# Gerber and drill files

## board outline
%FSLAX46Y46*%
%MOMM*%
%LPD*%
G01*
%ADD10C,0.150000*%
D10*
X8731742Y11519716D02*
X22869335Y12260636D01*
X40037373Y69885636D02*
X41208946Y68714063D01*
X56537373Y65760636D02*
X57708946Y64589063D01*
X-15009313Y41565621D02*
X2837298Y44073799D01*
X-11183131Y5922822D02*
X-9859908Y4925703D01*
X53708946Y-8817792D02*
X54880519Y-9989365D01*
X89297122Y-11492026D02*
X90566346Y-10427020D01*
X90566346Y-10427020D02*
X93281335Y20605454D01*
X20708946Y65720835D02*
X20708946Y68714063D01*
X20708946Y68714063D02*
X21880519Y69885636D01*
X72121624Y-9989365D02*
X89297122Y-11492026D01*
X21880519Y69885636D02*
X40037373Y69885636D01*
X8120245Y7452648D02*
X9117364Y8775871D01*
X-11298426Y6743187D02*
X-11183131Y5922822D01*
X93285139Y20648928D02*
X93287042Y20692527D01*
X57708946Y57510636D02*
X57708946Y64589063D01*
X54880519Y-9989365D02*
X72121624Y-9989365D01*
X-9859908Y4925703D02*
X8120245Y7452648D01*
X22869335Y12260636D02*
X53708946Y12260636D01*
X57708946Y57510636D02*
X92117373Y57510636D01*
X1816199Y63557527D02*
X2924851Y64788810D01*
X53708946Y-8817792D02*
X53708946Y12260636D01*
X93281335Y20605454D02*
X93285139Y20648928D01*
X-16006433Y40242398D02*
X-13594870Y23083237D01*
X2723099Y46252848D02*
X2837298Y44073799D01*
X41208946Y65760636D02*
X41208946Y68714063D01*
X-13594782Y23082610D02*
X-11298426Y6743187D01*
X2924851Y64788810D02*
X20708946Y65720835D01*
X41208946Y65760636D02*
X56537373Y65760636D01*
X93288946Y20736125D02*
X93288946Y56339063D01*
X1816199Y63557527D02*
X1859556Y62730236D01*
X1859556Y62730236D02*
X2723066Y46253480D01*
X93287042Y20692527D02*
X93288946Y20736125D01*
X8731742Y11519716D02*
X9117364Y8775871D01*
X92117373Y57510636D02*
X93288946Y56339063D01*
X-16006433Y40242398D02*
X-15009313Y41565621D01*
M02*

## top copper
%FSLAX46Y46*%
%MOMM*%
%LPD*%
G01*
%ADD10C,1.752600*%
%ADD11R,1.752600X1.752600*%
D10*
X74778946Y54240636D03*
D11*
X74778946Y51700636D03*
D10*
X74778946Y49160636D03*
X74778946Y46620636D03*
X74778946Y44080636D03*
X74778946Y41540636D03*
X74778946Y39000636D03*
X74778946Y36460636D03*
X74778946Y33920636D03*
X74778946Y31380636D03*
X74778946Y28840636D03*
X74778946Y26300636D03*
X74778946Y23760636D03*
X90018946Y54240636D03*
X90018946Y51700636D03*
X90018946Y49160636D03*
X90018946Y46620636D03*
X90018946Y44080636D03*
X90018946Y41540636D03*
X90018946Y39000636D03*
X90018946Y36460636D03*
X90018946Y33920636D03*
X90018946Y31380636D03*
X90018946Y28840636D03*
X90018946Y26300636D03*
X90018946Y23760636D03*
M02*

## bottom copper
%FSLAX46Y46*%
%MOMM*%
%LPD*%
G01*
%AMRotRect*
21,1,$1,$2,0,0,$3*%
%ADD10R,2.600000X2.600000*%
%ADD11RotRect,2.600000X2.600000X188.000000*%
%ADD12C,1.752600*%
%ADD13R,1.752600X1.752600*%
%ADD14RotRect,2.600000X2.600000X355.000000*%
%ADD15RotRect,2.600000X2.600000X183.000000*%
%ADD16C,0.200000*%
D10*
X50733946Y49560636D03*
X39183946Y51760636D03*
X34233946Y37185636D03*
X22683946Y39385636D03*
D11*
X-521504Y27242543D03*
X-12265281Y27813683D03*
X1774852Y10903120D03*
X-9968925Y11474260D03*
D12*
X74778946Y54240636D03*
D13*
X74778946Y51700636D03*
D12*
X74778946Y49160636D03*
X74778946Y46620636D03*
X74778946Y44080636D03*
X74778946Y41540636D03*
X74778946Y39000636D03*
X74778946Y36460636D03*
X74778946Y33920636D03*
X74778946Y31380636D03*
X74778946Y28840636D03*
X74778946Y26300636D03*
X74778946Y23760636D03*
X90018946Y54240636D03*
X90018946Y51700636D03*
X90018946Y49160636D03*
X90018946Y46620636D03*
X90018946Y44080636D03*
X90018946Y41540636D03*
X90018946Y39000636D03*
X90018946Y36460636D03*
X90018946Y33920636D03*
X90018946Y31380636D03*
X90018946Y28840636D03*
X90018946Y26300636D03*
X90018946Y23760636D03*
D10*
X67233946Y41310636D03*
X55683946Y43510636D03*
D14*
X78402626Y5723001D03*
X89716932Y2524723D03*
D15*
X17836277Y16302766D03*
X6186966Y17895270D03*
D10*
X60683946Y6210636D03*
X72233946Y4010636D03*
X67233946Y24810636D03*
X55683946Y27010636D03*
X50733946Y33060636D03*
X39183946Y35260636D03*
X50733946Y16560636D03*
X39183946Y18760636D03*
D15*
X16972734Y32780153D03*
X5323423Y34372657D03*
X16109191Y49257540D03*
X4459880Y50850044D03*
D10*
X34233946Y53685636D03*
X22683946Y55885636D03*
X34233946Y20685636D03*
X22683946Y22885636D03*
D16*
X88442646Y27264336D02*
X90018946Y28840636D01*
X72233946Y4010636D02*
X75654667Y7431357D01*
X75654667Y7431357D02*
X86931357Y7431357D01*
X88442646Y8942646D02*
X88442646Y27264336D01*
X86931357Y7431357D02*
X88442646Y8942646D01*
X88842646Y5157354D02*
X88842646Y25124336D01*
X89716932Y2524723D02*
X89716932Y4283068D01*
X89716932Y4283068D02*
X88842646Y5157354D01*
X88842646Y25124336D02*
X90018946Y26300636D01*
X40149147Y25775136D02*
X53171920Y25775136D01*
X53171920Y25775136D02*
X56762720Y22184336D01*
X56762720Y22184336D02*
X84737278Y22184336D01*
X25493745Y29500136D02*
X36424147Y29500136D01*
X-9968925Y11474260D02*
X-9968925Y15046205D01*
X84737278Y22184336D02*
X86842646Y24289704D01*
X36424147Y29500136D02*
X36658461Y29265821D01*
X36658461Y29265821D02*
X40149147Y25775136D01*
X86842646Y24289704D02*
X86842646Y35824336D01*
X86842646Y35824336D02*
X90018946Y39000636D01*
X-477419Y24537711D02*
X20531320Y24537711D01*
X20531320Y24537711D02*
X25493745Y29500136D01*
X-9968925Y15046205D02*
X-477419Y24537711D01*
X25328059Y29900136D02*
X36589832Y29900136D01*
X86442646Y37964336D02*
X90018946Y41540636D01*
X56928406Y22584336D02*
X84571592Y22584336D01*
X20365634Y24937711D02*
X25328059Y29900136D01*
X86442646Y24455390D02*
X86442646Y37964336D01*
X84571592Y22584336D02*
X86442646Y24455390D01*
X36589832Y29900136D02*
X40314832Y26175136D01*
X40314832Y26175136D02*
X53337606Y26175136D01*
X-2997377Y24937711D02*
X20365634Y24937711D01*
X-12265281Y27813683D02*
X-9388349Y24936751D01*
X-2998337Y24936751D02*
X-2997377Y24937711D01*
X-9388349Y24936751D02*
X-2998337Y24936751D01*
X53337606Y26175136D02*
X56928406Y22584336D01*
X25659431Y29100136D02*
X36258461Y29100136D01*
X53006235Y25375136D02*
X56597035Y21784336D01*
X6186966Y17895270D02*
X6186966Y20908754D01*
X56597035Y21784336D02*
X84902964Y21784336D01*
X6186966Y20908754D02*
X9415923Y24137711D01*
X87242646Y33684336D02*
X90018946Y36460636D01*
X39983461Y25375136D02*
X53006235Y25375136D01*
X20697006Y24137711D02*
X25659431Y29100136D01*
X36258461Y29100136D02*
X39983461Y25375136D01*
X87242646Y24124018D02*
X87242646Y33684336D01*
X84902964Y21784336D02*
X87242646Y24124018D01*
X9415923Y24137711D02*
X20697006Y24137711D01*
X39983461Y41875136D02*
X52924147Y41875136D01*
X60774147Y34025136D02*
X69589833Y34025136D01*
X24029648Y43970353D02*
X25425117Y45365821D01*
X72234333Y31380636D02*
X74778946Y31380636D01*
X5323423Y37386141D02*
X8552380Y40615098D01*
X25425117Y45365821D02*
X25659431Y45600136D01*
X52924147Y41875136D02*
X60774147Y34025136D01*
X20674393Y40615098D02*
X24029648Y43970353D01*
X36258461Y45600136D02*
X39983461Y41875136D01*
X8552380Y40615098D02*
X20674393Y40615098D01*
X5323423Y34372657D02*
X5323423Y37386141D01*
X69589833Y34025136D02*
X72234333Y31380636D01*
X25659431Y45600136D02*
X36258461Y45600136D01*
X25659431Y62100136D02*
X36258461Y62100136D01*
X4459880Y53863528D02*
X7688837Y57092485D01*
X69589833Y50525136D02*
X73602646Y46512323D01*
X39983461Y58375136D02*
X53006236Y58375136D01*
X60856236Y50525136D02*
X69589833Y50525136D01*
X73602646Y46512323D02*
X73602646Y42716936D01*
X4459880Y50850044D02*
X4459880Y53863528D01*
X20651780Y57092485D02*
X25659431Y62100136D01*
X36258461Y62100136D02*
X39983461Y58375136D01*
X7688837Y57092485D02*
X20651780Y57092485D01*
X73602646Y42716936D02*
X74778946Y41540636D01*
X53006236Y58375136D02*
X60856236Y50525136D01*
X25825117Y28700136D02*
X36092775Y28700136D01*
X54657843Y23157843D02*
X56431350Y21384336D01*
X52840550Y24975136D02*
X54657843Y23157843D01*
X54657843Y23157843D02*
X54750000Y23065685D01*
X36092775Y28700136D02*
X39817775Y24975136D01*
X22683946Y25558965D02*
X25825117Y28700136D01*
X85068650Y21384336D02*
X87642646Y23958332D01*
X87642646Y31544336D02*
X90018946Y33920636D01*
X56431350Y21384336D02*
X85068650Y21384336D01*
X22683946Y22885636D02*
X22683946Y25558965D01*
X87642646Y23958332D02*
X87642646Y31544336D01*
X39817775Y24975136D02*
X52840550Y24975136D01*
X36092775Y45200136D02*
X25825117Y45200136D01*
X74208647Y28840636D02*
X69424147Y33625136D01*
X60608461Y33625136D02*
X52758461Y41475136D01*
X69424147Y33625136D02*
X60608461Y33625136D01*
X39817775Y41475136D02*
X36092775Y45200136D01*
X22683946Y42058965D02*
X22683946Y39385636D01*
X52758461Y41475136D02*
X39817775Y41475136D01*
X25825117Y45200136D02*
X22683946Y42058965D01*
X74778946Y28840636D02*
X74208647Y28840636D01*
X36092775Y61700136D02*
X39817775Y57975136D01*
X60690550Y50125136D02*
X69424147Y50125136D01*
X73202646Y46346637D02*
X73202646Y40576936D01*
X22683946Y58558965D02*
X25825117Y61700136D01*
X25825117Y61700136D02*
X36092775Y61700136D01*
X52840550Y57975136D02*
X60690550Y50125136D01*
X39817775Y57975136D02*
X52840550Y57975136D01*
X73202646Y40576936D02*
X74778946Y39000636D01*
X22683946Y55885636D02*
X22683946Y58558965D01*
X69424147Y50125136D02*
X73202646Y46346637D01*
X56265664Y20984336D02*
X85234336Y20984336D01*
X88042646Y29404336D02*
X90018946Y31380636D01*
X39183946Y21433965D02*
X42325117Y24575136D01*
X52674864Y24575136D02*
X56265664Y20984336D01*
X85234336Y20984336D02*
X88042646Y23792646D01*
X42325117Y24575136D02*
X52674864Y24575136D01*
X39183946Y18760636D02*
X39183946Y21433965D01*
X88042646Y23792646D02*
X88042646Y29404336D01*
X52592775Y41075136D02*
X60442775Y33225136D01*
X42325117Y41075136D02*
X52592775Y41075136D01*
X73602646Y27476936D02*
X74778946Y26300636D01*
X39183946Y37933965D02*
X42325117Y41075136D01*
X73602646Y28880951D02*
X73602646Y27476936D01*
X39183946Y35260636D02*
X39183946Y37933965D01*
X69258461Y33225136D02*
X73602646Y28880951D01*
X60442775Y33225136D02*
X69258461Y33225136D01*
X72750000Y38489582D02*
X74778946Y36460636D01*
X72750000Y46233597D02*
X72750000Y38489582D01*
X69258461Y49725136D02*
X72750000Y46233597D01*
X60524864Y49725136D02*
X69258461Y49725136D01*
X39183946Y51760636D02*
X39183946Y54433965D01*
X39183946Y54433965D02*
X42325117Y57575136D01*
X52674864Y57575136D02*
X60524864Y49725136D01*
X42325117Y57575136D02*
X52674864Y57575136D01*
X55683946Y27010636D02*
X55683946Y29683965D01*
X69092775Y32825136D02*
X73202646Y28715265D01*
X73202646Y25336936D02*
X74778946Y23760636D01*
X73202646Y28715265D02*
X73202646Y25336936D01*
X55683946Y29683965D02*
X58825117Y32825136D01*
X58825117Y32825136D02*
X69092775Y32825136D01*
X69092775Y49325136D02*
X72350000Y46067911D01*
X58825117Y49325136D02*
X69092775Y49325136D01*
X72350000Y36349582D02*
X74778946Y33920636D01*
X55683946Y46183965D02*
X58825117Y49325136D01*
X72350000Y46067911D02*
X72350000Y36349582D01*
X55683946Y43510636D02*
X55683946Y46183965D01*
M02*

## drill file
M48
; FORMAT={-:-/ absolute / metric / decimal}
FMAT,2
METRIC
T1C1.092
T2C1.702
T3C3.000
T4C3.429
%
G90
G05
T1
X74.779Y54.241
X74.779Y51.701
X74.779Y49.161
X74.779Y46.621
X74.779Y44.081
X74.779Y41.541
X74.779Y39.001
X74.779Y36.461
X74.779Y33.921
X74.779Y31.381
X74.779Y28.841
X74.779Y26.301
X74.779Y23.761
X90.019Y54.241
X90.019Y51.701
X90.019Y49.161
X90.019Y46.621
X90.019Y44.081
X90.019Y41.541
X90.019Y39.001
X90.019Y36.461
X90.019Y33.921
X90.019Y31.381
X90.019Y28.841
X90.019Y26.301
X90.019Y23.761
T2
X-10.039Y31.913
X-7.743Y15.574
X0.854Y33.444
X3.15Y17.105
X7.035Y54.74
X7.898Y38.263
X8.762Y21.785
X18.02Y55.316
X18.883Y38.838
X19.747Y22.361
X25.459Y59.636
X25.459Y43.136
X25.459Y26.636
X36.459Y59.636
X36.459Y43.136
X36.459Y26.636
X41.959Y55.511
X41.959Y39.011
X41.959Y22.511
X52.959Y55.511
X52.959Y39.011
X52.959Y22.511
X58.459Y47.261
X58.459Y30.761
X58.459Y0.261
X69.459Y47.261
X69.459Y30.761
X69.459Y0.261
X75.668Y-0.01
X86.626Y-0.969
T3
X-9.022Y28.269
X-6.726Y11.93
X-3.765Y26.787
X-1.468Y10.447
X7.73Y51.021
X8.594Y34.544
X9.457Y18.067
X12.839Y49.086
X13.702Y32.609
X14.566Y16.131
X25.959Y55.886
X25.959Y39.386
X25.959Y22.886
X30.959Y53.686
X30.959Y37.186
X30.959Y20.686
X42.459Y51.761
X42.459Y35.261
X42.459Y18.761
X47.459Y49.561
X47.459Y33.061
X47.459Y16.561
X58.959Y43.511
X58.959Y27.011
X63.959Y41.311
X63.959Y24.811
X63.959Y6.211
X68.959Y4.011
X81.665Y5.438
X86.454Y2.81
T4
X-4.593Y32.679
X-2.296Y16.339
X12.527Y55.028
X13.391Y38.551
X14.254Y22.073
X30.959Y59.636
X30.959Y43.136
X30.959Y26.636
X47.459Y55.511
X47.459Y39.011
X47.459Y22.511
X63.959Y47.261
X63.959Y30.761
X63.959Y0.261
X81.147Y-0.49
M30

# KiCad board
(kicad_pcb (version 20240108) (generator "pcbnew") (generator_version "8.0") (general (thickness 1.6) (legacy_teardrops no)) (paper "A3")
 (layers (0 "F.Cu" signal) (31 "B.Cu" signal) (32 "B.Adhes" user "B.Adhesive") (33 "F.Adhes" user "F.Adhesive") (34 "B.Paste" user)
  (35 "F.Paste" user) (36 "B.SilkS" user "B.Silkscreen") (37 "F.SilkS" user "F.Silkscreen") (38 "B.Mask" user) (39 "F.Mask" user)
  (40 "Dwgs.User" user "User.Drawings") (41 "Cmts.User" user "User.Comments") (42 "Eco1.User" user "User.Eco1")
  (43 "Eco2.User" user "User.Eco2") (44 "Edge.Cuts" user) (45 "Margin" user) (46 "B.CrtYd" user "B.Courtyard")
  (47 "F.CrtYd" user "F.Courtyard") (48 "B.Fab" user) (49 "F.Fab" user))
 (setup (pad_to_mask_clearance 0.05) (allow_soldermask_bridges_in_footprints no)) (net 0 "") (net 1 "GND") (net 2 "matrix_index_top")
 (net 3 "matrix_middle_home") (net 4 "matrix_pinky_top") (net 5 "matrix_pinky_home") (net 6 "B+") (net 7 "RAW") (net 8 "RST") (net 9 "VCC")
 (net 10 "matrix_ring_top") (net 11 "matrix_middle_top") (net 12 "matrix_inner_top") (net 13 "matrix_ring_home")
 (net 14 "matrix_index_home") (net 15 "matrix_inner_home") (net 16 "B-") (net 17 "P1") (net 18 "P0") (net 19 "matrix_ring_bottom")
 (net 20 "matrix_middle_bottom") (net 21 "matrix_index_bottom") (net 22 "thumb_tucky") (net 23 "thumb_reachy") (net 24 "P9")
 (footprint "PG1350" (layer "F.Cu") (at 47.458946 -55.510636 180)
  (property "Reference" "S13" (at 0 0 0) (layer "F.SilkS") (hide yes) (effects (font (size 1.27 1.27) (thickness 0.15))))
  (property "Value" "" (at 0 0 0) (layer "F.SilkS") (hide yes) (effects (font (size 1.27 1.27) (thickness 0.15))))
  (pad "" np_thru_hole circle (at -5.5 0) (size 1.7018 1.7018) (drill 1.7018) (layers "*.Cu" "*.Mask"))
  (pad "" np_thru_hole circle (at 0 -5.95) (size 3 3) (drill 3) (layers "*.Cu" "*.Mask"))
  (pad "" np_thru_hole circle (at 0 0) (size 3.429 3.429) (drill 3.429) (layers "*.Cu" "*.Mask"))
  (pad "" np_thru_hole circle (at 5 -3.75) (size 3 3) (drill 3) (layers "*.Cu" "*.Mask"))
  (pad "" np_thru_hole circle (at 5.5 0) (size 1.7018 1.7018) (drill 1.7018) (layers "*.Cu" "*.Mask"))
  (pad "1" smd rect (at -3.275 -5.95 180) (size 2.6 2.6) (layers "B.Cu" "B.Paste" "B.Mask") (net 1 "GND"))
  (pad "2" smd rect (at 8.275 -3.75 180) (size 2.6 2.6) (layers "B.Cu" "B.Paste" "B.Mask") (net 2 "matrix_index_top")))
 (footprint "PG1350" (layer "F.Cu") (at 30.958946 -43.135636 180)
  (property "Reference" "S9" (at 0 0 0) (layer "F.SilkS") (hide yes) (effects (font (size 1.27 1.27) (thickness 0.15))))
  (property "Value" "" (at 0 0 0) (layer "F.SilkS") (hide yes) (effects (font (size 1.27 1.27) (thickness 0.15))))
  (pad "" np_thru_hole circle (at -5.5 0) (size 1.7018 1.7018) (drill 1.7018) (layers "*.Cu" "*.Mask"))
  (pad "" np_thru_hole circle (at 0 -5.95) (size 3 3) (drill 3) (layers "*.Cu" "*.Mask"))
  (pad "" np_thru_hole circle (at 0 0) (size 3.429 3.429) (drill 3.429) (layers "*.Cu" "*.Mask"))
  (pad "" np_thru_hole circle (at 5 -3.75) (size 3 3) (drill 3) (layers "*.Cu" "*.Mask"))
  (pad "" np_thru_hole circle (at 5.5 0) (size 1.7018 1.7018) (drill 1.7018) (layers "*.Cu" "*.Mask"))
  (pad "1" smd rect (at -3.275 -5.95 180) (size 2.6 2.6) (layers "B.Cu" "B.Paste" "B.Mask") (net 1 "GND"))
  (pad "2" smd rect (at 8.275 -3.75 180) (size 2.6 2.6) (layers "B.Cu" "B.Paste" "B.Mask") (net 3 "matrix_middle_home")))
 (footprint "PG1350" (layer "F.Cu") (at -4.592712 -32.678846 -172)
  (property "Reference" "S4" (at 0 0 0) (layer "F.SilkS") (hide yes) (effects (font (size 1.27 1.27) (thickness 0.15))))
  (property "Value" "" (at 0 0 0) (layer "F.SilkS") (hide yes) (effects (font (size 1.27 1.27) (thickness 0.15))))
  (pad "" np_thru_hole circle (at -5.5 0) (size 1.7018 1.7018) (drill 1.7018) (layers "*.Cu" "*.Mask"))
  (pad "" np_thru_hole circle (at 0 -5.95) (size 3 3) (drill 3) (layers "*.Cu" "*.Mask"))
  (pad "" np_thru_hole circle (at 0 0) (size 3.429 3.429) (drill 3.429) (layers "*.Cu" "*.Mask"))
  (pad "" np_thru_hole circle (at 5 -3.75) (size 3 3) (drill 3) (layers "*.Cu" "*.Mask"))
  (pad "" np_thru_hole circle (at 5.5 0) (size 1.7018 1.7018) (drill 1.7018) (layers "*.Cu" "*.Mask"))
  (pad "1" smd rect (at -3.275 -5.95 188) (size 2.6 2.6) (layers "B.Cu" "B.Paste" "B.Mask") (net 1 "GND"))
  (pad "2" smd rect (at 8.275 -3.75 188) (size 2.6 2.6) (layers "B.Cu" "B.Paste" "B.Mask") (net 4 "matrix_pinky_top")))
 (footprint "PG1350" (layer "F.Cu") (at -2.296356 -16.339423 -172)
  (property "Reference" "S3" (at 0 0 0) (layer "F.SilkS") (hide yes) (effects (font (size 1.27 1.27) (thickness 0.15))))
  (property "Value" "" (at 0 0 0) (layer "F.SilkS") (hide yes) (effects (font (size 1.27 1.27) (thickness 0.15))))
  (pad "" np_thru_hole circle (at -5.5 0) (size 1.7018 1.7018) (drill 1.7018) (layers "*.Cu" "*.Mask"))
  (pad "" np_thru_hole circle (at 0 -5.95) (size 3 3) (drill 3) (layers "*.Cu" "*.Mask"))
  (pad "" np_thru_hole circle (at 0 0) (size 3.429 3.429) (drill 3.429) (layers "*.Cu" "*.Mask"))
  (pad "" np_thru_hole circle (at 5 -3.75) (size 3 3) (drill 3) (layers "*.Cu" "*.Mask"))
  (pad "" np_thru_hole circle (at 5.5 0) (size 1.7018 1.7018) (drill 1.7018) (layers "*.Cu" "*.Mask"))
  (pad "1" smd rect (at -3.275 -5.95 188) (size 2.6 2.6) (layers "B.Cu" "B.Paste" "B.Mask") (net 1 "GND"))
  (pad "2" smd rect (at 8.275 -3.75 188) (size 2.6 2.6) (layers "B.Cu" "B.Paste" "B.Mask") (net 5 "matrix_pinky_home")))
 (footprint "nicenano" (layer "F.Cu") (at 82.398946 -39.000636 -90)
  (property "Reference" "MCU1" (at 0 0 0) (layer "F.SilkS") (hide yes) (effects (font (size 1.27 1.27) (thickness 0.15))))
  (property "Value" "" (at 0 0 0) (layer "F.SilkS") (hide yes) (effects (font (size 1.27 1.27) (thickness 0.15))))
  (pad "1" thru_hole circle (at -15.24 7.62) (size 1.7526 1.7526) (drill 1.0922) (layers "*.Cu" "*.SilkS" "*.Mask")
   (remove_unused_layers no) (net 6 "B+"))
  (pad "2" thru_hole rect (at -12.7 7.62 270) (size 1.7526 1.7526) (drill 1.0922) (layers "*.Cu" "*.SilkS" "*.Mask")
   (remove_unused_layers no) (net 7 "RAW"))
  (pad "3" thru_hole circle (at -10.16 7.62) (size 1.7526 1.7526) (drill 1.0922) (layers "*.Cu" "*.SilkS" "*.Mask")
   (remove_unused_layers no) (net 1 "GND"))
  (pad "4" thru_hole circle (at -7.62 7.62) (size 1.7526 1.7526) (drill 1.0922) (layers "*.Cu" "*.SilkS" "*.Mask") (remove_unused_layers no)
   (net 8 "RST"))
  (pad "5" thru_hole circle (at -5.08 7.62) (size 1.7526 1.7526) (drill 1.0922) (layers "*.Cu" "*.SilkS" "*.Mask") (remove_unused_layers no)
   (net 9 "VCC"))
  (pad "6" thru_hole circle (at -2.54 7.62) (size 1.7526 1.7526) (drill 1.0922) (layers "*.Cu" "*.SilkS" "*.Mask") (remove_unused_layers no)
   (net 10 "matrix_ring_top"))
  (pad "7" thru_hole circle (at 0 7.62) (size 1.7526 1.7526) (drill 1.0922) (layers "*.Cu" "*.SilkS" "*.Mask") (remove_unused_layers no)
   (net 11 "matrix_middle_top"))
  (pad "8" thru_hole circle (at 2.54 7.62) (size 1.7526 1.7526) (drill 1.0922) (layers "*.Cu" "*.SilkS" "*.Mask") (remove_unused_layers no)
   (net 2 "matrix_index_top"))
  (pad "9" thru_hole circle (at 5.08 7.62) (size 1.7526 1.7526) (drill 1.0922) (layers "*.Cu" "*.SilkS" "*.Mask") (remove_unused_layers no)
   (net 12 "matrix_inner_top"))
  (pad "10" thru_hole circle (at 7.62 7.62) (size 1.7526 1.7526) (drill 1.0922) (layers "*.Cu" "*.SilkS" "*.Mask") (remove_unused_layers no)
   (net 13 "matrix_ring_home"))
  (pad "11" thru_hole circle (at 10.16 7.62) (size 1.7526 1.7526) (drill 1.0922) (layers "*.Cu" "*.SilkS" "*.Mask")
   (remove_unused_layers no) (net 3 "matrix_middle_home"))
  (pad "12" thru_hole circle (at 12.7 7.62) (size 1.7526 1.7526) (drill 1.0922) (layers "*.Cu" "*.SilkS" "*.Mask") (remove_unused_layers no)
   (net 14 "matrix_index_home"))
  (pad "13" thru_hole circle (at 15.24 7.62) (size 1.7526 1.7526) (drill 1.0922) (layers "*.Cu" "*.SilkS" "*.Mask")
   (remove_unused_layers no) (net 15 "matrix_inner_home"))
  (pad "14" thru_hole circle (at -15.24 -7.62) (size 1.7526 1.7526) (drill 1.0922) (layers "*.Cu" "*.SilkS" "*.Mask")
   (remove_unused_layers no) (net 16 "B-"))
  (pad "15" thru_hole circle (at -12.7 -7.62) (size 1.7526 1.7526) (drill 1.0922) (layers "*.Cu" "*.SilkS" "*.Mask")
   (remove_unused_layers no) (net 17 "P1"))
  (pad "16" thru_hole circle (at -10.16 -7.62) (size 1.7526 1.7526) (drill 1.0922) (layers "*.Cu" "*.SilkS" "*.Mask")
   (remove_unused_layers no) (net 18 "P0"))
  (pad "17" thru_hole circle (at -7.62 -7.62) (size 1.7526 1.7526) (drill 1.0922) (layers "*.Cu" "*.SilkS" "*.Mask")
   (remove_unused_layers no) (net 1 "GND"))
  (pad "18" thru_hole circle (at -5.08 -7.62) (size 1.7526 1.7526) (drill 1.0922) (layers "*.Cu" "*.SilkS" "*.Mask")
   (remove_unused_layers no) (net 1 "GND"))
  (pad "19" thru_hole circle (at -2.54 -7.62) (size 1.7526 1.7526) (drill 1.0922) (layers "*.Cu" "*.SilkS" "*.Mask")
   (remove_unused_layers no) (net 4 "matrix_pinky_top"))
  (pad "20" thru_hole circle (at 0 -7.62) (size 1.7526 1.7526) (drill 1.0922) (layers "*.Cu" "*.SilkS" "*.Mask") (remove_unused_layers no)
   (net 5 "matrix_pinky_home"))
  (pad "21" thru_hole circle (at 2.54 -7.62) (size 1.7526 1.7526) (drill 1.0922) (layers "*.Cu" "*.SilkS" "*.Mask")
   (remove_unused_layers no) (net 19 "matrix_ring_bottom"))
  (pad "22" thru_hole circle (at 5.08 -7.62) (size 1.7526 1.7526) (drill 1.0922) (layers "*.Cu" "*.SilkS" "*.Mask")
   (remove_unused_layers no) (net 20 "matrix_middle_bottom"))
  (pad "23" thru_hole circle (at 7.62 -7.62) (size 1.7526 1.7526) (drill 1.0922) (layers "*.Cu" "*.SilkS" "*.Mask")
   (remove_unused_layers no) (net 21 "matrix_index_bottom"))
  (pad "24" thru_hole circle (at 10.16 -7.62) (size 1.7526 1.7526) (drill 1.0922) (layers "*.Cu" "*.SilkS" "*.Mask")
   (remove_unused_layers no) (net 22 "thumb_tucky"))
  (pad "25" thru_hole circle (at 12.7 -7.62) (size 1.7526 1.7526) (drill 1.0922) (layers "*.Cu" "*.SilkS" "*.Mask")
   (remove_unused_layers no) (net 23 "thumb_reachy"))
  (pad "26" thru_hole circle (at 15.24 -7.62) (size 1.7526 1.7526) (drill 1.0922) (layers "*.Cu" "*.SilkS" "*.Mask")
   (remove_unused_layers no) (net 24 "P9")))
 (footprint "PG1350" (layer "F.Cu") (at 63.958946 -47.260636 180)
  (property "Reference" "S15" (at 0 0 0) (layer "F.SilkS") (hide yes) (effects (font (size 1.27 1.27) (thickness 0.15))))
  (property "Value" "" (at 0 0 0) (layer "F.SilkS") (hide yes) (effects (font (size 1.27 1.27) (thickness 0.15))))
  (pad "" np_thru_hole circle (at -5.5 0) (size 1.7018 1.7018) (drill 1.7018) (layers "*.Cu" "*.Mask"))
  (pad "" np_thru_hole circle (at 0 -5.95) (size 3 3) (drill 3) (layers "*.Cu" "*.Mask"))
  (pad "" np_thru_hole circle (at 0 0) (size 3.429 3.429) (drill 3.429) (layers "*.Cu" "*.Mask"))
  (pad "" np_thru_hole circle (at 5 -3.75) (size 3 3) (drill 3) (layers "*.Cu" "*.Mask"))
  (pad "" np_thru_hole circle (at 5.5 0) (size 1.7018 1.7018) (drill 1.7018) (layers "*.Cu" "*.Mask"))
  (pad "1" smd rect (at -3.275 -5.95 180) (size 2.6 2.6) (layers "B.Cu" "B.Paste" "B.Mask") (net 1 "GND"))
  (pad "2" smd rect (at 8.275 -3.75 180) (size 2.6 2.6) (layers "B.Cu" "B.Paste" "B.Mask") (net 12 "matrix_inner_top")))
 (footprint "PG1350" (layer "F.Cu") (at 81.146587 0.489793 -5)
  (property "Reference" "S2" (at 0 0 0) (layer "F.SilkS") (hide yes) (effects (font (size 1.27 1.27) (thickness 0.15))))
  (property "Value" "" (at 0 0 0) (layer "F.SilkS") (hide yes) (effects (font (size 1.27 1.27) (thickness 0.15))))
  (pad "" np_thru_hole circle (at -5.5 0) (size 1.7018 1.7018) (drill 1.7018) (layers "*.Cu" "*.Mask"))
  (pad "" np_thru_hole circle (at 0 -5.95) (size 3 3) (drill 3) (layers "*.Cu" "*.Mask"))
  (pad "" np_thru_hole circle (at 0 0) (size 3.429 3.429) (drill 3.429) (layers "*.Cu" "*.Mask"))
  (pad "" np_thru_hole circle (at 5.000001 -3.75) (size 3 3) (drill 3) (layers "*.Cu" "*.Mask"))
  (pad "" np_thru_hole circle (at 5.5 0) (size 1.7018 1.7018) (drill 1.7018) (layers "*.Cu" "*.Mask"))
  (pad "1" smd rect (at -3.275 -5.95 355) (size 2.6 2.6) (layers "B.Cu" "B.Paste" "B.Mask") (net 1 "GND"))
  (pad "2" smd rect (at 8.275 -3.75 355) (size 2.6 2.6) (layers "B.Cu" "B.Paste" "B.Mask") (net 23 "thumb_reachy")))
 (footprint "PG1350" (layer "F.Cu") (at 14.254366 -22.073211 -177)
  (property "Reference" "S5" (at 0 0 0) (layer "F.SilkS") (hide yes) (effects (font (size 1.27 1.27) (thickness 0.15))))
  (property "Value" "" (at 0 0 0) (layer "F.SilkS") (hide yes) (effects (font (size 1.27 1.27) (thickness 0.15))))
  (pad "" np_thru_hole circle (at -5.5 0) (size 1.7018 1.7018) (drill 1.7018) (layers "*.Cu" "*.Mask"))
  (pad "" np_thru_hole circle (at 0 -5.95) (size 3 3) (drill 3) (layers "*.Cu" "*.Mask"))
  (pad "" np_thru_hole circle (at 0 0) (size 3.429 3.429) (drill 3.429) (layers "*.Cu" "*.Mask"))
  (pad "" np_thru_hole circle (at 5 -3.75) (size 3 3) (drill 3) (layers "*.Cu" "*.Mask"))
  (pad "" np_thru_hole circle (at 5.5 0) (size 1.7018 1.7018) (drill 1.7018) (layers "*.Cu" "*.Mask"))
  (pad "1" smd rect (at -3.275 -5.95 183) (size 2.6 2.6) (layers "B.Cu" "B.Paste" "B.Mask") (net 1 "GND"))
  (pad "2" smd rect (at 8.275 -3.75 183) (size 2.6 2.6) (layers "B.Cu" "B.Paste" "B.Mask") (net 19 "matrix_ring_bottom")))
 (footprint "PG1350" (layer "F.Cu") (at 63.958946 -0.260636)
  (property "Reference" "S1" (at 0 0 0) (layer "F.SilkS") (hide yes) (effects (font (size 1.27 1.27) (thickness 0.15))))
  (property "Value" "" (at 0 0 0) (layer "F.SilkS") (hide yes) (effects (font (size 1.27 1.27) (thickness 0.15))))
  (pad "" np_thru_hole circle (at -5.5 0) (size 1.7018 1.7018) (drill 1.7018) (layers "*.Cu" "*.Mask"))
  (pad "" np_thru_hole circle (at 0 -5.95) (size 3 3) (drill 3) (layers "*.Cu" "*.Mask"))
  (pad "" np_thru_hole circle (at 0 0) (size 3.429 3.429) (drill 3.429) (layers "*.Cu" "*.Mask"))
  (pad "" np_thru_hole circle (at 5 -3.75) (size 3 3) (drill 3) (layers "*.Cu" "*.Mask"))
  (pad "" np_thru_hole circle (at 5.5 0) (size 1.7018 1.7018) (drill 1.7018) (layers "*.Cu" "*.Mask"))
  (pad "1" smd rect (at -3.275 -5.95) (size 2.6 2.6) (layers "B.Cu" "B.Paste" "B.Mask") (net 1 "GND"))
  (pad "2" smd rect (at 8.275 -3.75) (size 2.6 2.6) (layers "B.Cu" "B.Paste" "B.Mask") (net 22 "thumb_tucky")))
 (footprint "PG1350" (layer "F.Cu") (at 63.958946 -30.760636 180)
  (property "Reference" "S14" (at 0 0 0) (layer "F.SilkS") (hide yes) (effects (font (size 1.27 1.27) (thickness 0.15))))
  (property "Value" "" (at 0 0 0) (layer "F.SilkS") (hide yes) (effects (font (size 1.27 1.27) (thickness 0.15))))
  (pad "" np_thru_hole circle (at -5.5 0) (size 1.7018 1.7018) (drill 1.7018) (layers "*.Cu" "*.Mask"))
  (pad "" np_thru_hole circle (at 0 -5.95) (size 3 3) (drill 3) (layers "*.Cu" "*.Mask"))
  (pad "" np_thru_hole circle (at 0 0) (size 3.429 3.429) (drill 3.429) (layers "*.Cu" "*.Mask"))
  (pad "" np_thru_hole circle (at 5 -3.75) (size 3 3) (drill 3) (layers "*.Cu" "*.Mask"))
  (pad "" np_thru_hole circle (at 5.5 0) (size 1.7018 1.7018) (drill 1.7018) (layers "*.Cu" "*.Mask"))
  (pad "1" smd rect (at -3.275 -5.95 180) (size 2.6 2.6) (layers "B.Cu" "B.Paste" "B.Mask") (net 1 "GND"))
  (pad "2" smd rect (at 8.275 -3.75 180) (size 2.6 2.6) (layers "B.Cu" "B.Paste" "B.Mask") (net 15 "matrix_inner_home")))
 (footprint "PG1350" (layer "F.Cu") (at 47.458946 -39.010636 180)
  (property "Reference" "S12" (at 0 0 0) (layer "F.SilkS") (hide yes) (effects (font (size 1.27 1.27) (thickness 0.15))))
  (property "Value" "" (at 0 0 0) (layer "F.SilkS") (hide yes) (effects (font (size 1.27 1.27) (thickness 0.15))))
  (pad "" np_thru_hole circle (at -5.5 0) (size 1.7018 1.7018) (drill 1.7018) (layers "*.Cu" "*.Mask"))
  (pad "" np_thru_hole circle (at 0 -5.95) (size 3 3) (drill 3) (layers "*.Cu" "*.Mask"))
  (pad "" np_thru_hole circle (at 0 0) (size 3.429 3.429) (drill 3.429) (layers "*.Cu" "*.Mask"))
  (pad "" np_thru_hole circle (at 5 -3.75) (size 3 3) (drill 3) (layers "*.Cu" "*.Mask"))
  (pad "" np_thru_hole circle (at 5.5 0) (size 1.7018 1.7018) (drill 1.7018) (layers "*.Cu" "*.Mask"))
  (pad "1" smd rect (at -3.275 -5.95 180) (size 2.6 2.6) (layers "B.Cu" "B.Paste" "B.Mask") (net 1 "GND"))
  (pad "2" smd rect (at 8.275 -3.75 180) (size 2.6 2.6) (layers "B.Cu" "B.Paste" "B.Mask") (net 14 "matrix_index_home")))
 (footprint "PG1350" (layer "F.Cu") (at 47.458946 -22.510636 180)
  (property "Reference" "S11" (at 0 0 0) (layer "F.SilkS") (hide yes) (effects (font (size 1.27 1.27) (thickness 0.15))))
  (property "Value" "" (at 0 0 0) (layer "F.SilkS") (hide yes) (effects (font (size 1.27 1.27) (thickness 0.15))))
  (pad "" np_thru_hole circle (at -5.5 0) (size 1.7018 1.7018) (drill 1.7018) (layers "*.Cu" "*.Mask"))
  (pad "" np_thru_hole circle (at 0 -5.95) (size 3 3) (drill 3) (layers "*.Cu" "*.Mask"))
  (pad "" np_thru_hole circle (at 0 0) (size 3.429 3.429) (drill 3.429) (layers "*.Cu" "*.Mask"))
  (pad "" np_thru_hole circle (at 5 -3.75) (size 3 3) (drill 3) (layers "*.Cu" "*.Mask"))
  (pad "" np_thru_hole circle (at 5.5 0) (size 1.7018 1.7018) (drill 1.7018) (layers "*.Cu" "*.Mask"))
  (pad "1" smd rect (at -3.275 -5.95 180) (size 2.6 2.6) (layers "B.Cu" "B.Paste" "B.Mask") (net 1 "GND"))
  (pad "2" smd rect (at 8.275 -3.75 180) (size 2.6 2.6) (layers "B.Cu" "B.Paste" "B.Mask") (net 21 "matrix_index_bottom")))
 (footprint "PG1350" (layer "F.Cu") (at 13.390823 -38.550598 -177)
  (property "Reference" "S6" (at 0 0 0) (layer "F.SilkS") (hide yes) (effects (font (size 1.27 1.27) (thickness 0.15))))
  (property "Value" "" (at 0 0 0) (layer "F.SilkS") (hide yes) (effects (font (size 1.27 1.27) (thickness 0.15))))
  (pad "" np_thru_hole circle (at -5.5 0) (size 1.7018 1.7018) (drill 1.7018) (layers "*.Cu" "*.Mask"))
  (pad "" np_thru_hole circle (at 0 -5.95) (size 3 3) (drill 3) (layers "*.Cu" "*.Mask"))
  (pad "" np_thru_hole circle (at 0 0) (size 3.429 3.429) (drill 3.429) (layers "*.Cu" "*.Mask"))
  (pad "" np_thru_hole circle (at 5 -3.75) (size 3 3) (drill 3) (layers "*.Cu" "*.Mask"))
  (pad "" np_thru_hole circle (at 5.5 0) (size 1.7018 1.7018) (drill 1.7018) (layers "*.Cu" "*.Mask"))
  (pad "1" smd rect (at -3.275 -5.95 183) (size 2.6 2.6) (layers "B.Cu" "B.Paste" "B.Mask") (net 1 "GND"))
  (pad "2" smd rect (at 8.275 -3.75 183) (size 2.6 2.6) (layers "B.Cu" "B.Paste" "B.Mask") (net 13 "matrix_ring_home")))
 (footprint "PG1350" (layer "F.Cu") (at 12.52728 -55.027985 -177)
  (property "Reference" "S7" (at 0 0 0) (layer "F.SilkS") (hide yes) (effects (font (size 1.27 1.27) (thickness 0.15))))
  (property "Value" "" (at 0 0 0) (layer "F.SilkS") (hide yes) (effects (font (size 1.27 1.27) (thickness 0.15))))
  (pad "" np_thru_hole circle (at -5.5 0) (size 1.7018 1.7018) (drill 1.7018) (layers "*.Cu" "*.Mask"))
  (pad "" np_thru_hole circle (at 0 -5.95) (size 3 3) (drill 3) (layers "*.Cu" "*.Mask"))
  (pad "" np_thru_hole circle (at 0 0) (size 3.429 3.429) (drill 3.429) (layers "*.Cu" "*.Mask"))
  (pad "" np_thru_hole circle (at 5 -3.75) (size 3 3) (drill 3) (layers "*.Cu" "*.Mask"))
  (pad "" np_thru_hole circle (at 5.5 0) (size 1.7018 1.7018) (drill 1.7018) (layers "*.Cu" "*.Mask"))
  (pad "1" smd rect (at -3.275 -5.95 183) (size 2.6 2.6) (layers "B.Cu" "B.Paste" "B.Mask") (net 1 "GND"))
  (pad "2" smd rect (at 8.275 -3.75 183) (size 2.6 2.6) (layers "B.Cu" "B.Paste" "B.Mask") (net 10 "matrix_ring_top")))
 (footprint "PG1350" (layer "F.Cu") (at 30.958946 -59.635636 180)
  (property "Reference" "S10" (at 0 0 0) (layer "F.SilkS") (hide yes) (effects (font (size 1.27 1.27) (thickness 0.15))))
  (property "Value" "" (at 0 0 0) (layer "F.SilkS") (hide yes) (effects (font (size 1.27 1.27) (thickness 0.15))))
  (pad "" np_thru_hole circle (at -5.5 0) (size 1.7018 1.7018) (drill 1.7018) (layers "*.Cu" "*.Mask"))
  (pad "" np_thru_hole circle (at 0 -5.95) (size 3 3) (drill 3) (layers "*.Cu" "*.Mask"))
  (pad "" np_thru_hole circle (at 0 0) (size 3.429 3.429) (drill 3.429) (layers "*.Cu" "*.Mask"))
  (pad "" np_thru_hole circle (at 5 -3.75) (size 3 3) (drill 3) (layers "*.Cu" "*.Mask"))
  (pad "" np_thru_hole circle (at 5.5 0) (size 1.7018 1.7018) (drill 1.7018) (layers "*.Cu" "*.Mask"))
  (pad "1" smd rect (at -3.275 -5.95 180) (size 2.6 2.6) (layers "B.Cu" "B.Paste" "B.Mask") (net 1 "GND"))
  (pad "2" smd rect (at 8.275 -3.75 180) (size 2.6 2.6) (layers "B.Cu" "B.Paste" "B.Mask") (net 11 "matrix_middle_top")))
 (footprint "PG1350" (layer "F.Cu") (at 30.958946 -26.635636 180)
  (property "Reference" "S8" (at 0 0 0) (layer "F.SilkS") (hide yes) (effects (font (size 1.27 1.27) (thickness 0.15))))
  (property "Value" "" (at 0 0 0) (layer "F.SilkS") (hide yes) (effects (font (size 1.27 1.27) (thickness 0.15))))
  (pad "" np_thru_hole circle (at -5.5 0) (size 1.7018 1.7018) (drill 1.7018) (layers "*.Cu" "*.Mask"))
  (pad "" np_thru_hole circle (at 0 -5.95) (size 3 3) (drill 3) (layers "*.Cu" "*.Mask"))
  (pad "" np_thru_hole circle (at 0 0) (size 3.429 3.429) (drill 3.429) (layers "*.Cu" "*.Mask"))
  (pad "" np_thru_hole circle (at 5 -3.75) (size 3 3) (drill 3) (layers "*.Cu" "*.Mask"))
  (pad "" np_thru_hole circle (at 5.5 0) (size 1.7018 1.7018) (drill 1.7018) (layers "*.Cu" "*.Mask"))
  (pad "1" smd rect (at -3.275 -5.95 180) (size 2.6 2.6) (layers "B.Cu" "B.Paste" "B.Mask") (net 1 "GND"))
  (pad "2" smd rect (at 8.275 -3.75 180) (size 2.6 2.6) (layers "B.Cu" "B.Paste" "B.Mask") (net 20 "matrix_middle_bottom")))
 (gr_line (start 8.731742 -11.519716) (end 22.869335 -12.260636) (stroke (width 0.15) (type default)) (layer "Edge.Cuts"))
 (gr_line (start 40.037373 -69.885636) (end 41.208946 -68.714063) (stroke (width 0.15) (type default)) (layer "Edge.Cuts"))
 (gr_line (start 56.537373 -65.760636) (end 57.708946 -64.589063) (stroke (width 0.15) (type default)) (layer "Edge.Cuts"))
 (gr_line (start -15.009313 -41.565621) (end 2.837298 -44.073799) (stroke (width 0.15) (type default)) (layer "Edge.Cuts"))
 (gr_line (start -11.183131 -5.922822) (end -9.859908 -4.925703) (stroke (width 0.15) (type default)) (layer "Edge.Cuts"))
 (gr_line (start 53.708946 8.817792) (end 54.880519 9.989365) (stroke (width 0.15) (type default)) (layer "Edge.Cuts"))
 (gr_line (start 89.297122 11.492026) (end 90.566346 10.42702) (stroke (width 0.15) (type default)) (layer "Edge.Cuts"))
 (gr_line (start 90.566346 10.42702) (end 93.281335 -20.605454) (stroke (width 0.15) (type default)) (layer "Edge.Cuts"))
 (gr_line (start 20.708946 -65.720835) (end 20.708946 -68.714063) (stroke (width 0.15) (type default)) (layer "Edge.Cuts"))
 (gr_line (start 20.708946 -68.714063) (end 21.880519 -69.885636) (stroke (width 0.15) (type default)) (layer "Edge.Cuts"))
 (gr_line (start 72.121624 9.989365) (end 89.297122 11.492026) (stroke (width 0.15) (type default)) (layer "Edge.Cuts"))
 (gr_line (start 21.880519 -69.885636) (end 40.037373 -69.885636) (stroke (width 0.15) (type default)) (layer "Edge.Cuts"))
 (gr_line (start 8.120245 -7.452648) (end 9.117364 -8.775871) (stroke (width 0.15) (type default)) (layer "Edge.Cuts"))
 (gr_line (start -11.298426 -6.743187) (end -11.183131 -5.922822) (stroke (width 0.15) (type default)) (layer "Edge.Cuts"))
 (gr_line (start 93.285139 -20.648928) (end 93.287042 -20.692527) (stroke (width 0.15) (type default)) (layer "Edge.Cuts"))
 (gr_line (start 57.708946 -57.510636) (end 57.708946 -64.589063) (stroke (width 0.15) (type default)) (layer "Edge.Cuts"))
 (gr_line (start 54.880519 9.989365) (end 72.121624 9.989365) (stroke (width 0.15) (type default)) (layer "Edge.Cuts"))
 (gr_line (start -9.859908 -4.925703) (end 8.120245 -7.452648) (stroke (width 0.15) (type default)) (layer "Edge.Cuts"))
 (gr_line (start 22.869335 -12.260636) (end 53.708946 -12.260636) (stroke (width 0.15) (type default)) (layer "Edge.Cuts"))
 (gr_line (start 57.708946 -57.510636) (end 92.117373 -57.510636) (stroke (width 0.15) (type default)) (layer "Edge.Cuts"))
 (gr_line (start 1.816199 -63.557527) (end 2.924851 -64.78881) (stroke (width 0.15) (type default)) (layer "Edge.Cuts"))
 (gr_line (start 53.708946 8.817792) (end 53.708946 -12.260636) (stroke (width 0.15) (type default)) (layer "Edge.Cuts"))
 (gr_line (start 93.281335 -20.605454) (end 93.285139 -20.648928) (stroke (width 0.15) (type default)) (layer "Edge.Cuts"))
 (gr_line (start -16.006433 -40.242398) (end -13.59487 -23.083237) (stroke (width 0.15) (type default)) (layer "Edge.Cuts"))
 (gr_line (start 2.723099 -46.252848) (end 2.837298 -44.073799) (stroke (width 0.15) (type default)) (layer "Edge.Cuts"))
 (gr_line (start 41.208946 -65.760636) (end 41.208946 -68.714063) (stroke (width 0.15) (type default)) (layer "Edge.Cuts"))
 (gr_line (start -13.594782 -23.08261) (end -11.298426 -6.743187) (stroke (width 0.15) (type default)) (layer "Edge.Cuts"))
 (gr_line (start 2.924851 -64.78881) (end 20.708946 -65.720835) (stroke (width 0.15) (type default)) (layer "Edge.Cuts"))
 (gr_line (start 41.208946 -65.760636) (end 56.537373 -65.760636) (stroke (width 0.15) (type default)) (layer "Edge.Cuts"))
 (gr_line (start 93.288946 -20.736125) (end 93.288946 -56.339063) (stroke (width 0.15) (type default)) (layer "Edge.Cuts"))
 (gr_line (start 1.816199 -63.557527) (end 1.859556 -62.730236) (stroke (width 0.15) (type default)) (layer "Edge.Cuts"))
 (gr_line (start 1.859556 -62.730236) (end 2.723066 -46.25348) (stroke (width 0.15) (type default)) (layer "Edge.Cuts"))
 (gr_line (start 93.287042 -20.692527) (end 93.288946 -20.736125) (stroke (width 0.15) (type default)) (layer "Edge.Cuts"))
 (gr_line (start 8.731742 -11.519716) (end 9.117364 -8.775871) (stroke (width 0.15) (type default)) (layer "Edge.Cuts"))
 (gr_line (start 92.117373 -57.510636) (end 93.288946 -56.339063) (stroke (width 0.15) (type default)) (layer "Edge.Cuts"))
 (gr_line (start -16.006433 -40.242398) (end -15.009313 -41.565621) (stroke (width 0.15) (type default)) (layer "Edge.Cuts"))
 (segment (start 88.442646 -27.264336) (end 90.018946 -28.840636) (width 0.2) (layer "B.Cu") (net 22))
 (segment (start 72.233946 -4.010636) (end 75.654667 -7.431357) (width 0.2) (layer "B.Cu") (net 22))
 (segment (start 75.654667 -7.431357) (end 86.931357 -7.431357) (width 0.2) (layer "B.Cu") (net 22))
 (segment (start 88.442646 -8.942646) (end 88.442646 -27.264336) (width 0.2) (layer "B.Cu") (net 22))
 (segment (start 86.931357 -7.431357) (end 88.442646 -8.942646) (width 0.2) (layer "B.Cu") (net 22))
 (segment (start 88.842646 -5.157354) (end 88.842646 -25.124336) (width 0.2) (layer "B.Cu") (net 23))
 (segment (start 89.716932 -2.524723) (end 89.716932 -4.283068) (width 0.2) (layer "B.Cu") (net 23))
 (segment (start 89.716932 -4.283068) (end 88.842646 -5.157354) (width 0.2) (layer "B.Cu") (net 23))
 (segment (start 88.842646 -25.124336) (end 90.018946 -26.300636) (width 0.2) (layer "B.Cu") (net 23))
 (segment (start 40.149147 -25.775136) (end 53.17192 -25.775136) (width 0.2) (layer "B.Cu") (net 5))
 (segment (start 53.17192 -25.775136) (end 56.76272 -22.184336) (width 0.2) (layer "B.Cu") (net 5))
 (segment (start 56.76272 -22.184336) (end 84.737278 -22.184336) (width 0.2) (layer "B.Cu") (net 5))
 (segment (start 25.493745 -29.500136) (end 36.424147 -29.500136) (width 0.2) (layer "B.Cu") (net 5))
 (segment (start -9.968925 -11.47426) (end -9.968925 -15.046205) (width 0.2) (layer "B.Cu") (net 5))
 (segment (start 84.737278 -22.184336) (end 86.842646 -24.289704) (width 0.2) (layer "B.Cu") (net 5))
 (segment (start 36.424147 -29.500136) (end 36.658461 -29.265821) (width 0.2) (layer "B.Cu") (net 5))
 (segment (start 36.658461 -29.265821) (end 40.149147 -25.775136) (width 0.2) (layer "B.Cu") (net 5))
 (segment (start 86.842646 -24.289704) (end 86.842646 -35.824336) (width 0.2) (layer "B.Cu") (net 5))
 (segment (start 86.842646 -35.824336) (end 90.018946 -39.000636) (width 0.2) (layer "B.Cu") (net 5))
 (segment (start -0.477419 -24.537711) (end 20.53132 -24.537711) (width 0.2) (layer "B.Cu") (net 5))
 (segment (start 20.53132 -24.537711) (end 25.493745 -29.500136) (width 0.2) (layer "B.Cu") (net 5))
 (segment (start -9.968925 -15.046205) (end -0.477419 -24.537711) (width 0.2) (layer "B.Cu") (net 5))
 (segment (start 25.328059 -29.900136) (end 36.589832 -29.900136) (width 0.2) (layer "B.Cu") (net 4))
 (segment (start 86.442646 -37.964336) (end 90.018946 -41.540636) (width 0.2) (layer "B.Cu") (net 4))
 (segment (start 56.928406 -22.584336) (end 84.571592 -22.584336) (width 0.2) (layer "B.Cu") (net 4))
 (segment (start 20.365634 -24.937711) (end 25.328059 -29.900136) (width 0.2) (layer "B.Cu") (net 4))
 (segment (start 86.442646 -24.45539) (end 86.442646 -37.964336) (width 0.2) (layer "B.Cu") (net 4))
 (segment (start 84.571592 -22.584336) (end 86.442646 -24.45539) (width 0.2) (layer "B.Cu") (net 4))
 (segment (start 36.589832 -29.900136) (end 40.314832 -26.175136) (width 0.2) (layer "B.Cu") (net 4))
 (segment (start 40.314832 -26.175136) (end 53.337606 -26.175136) (width 0.2) (layer "B.Cu") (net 4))
 (segment (start -2.997377 -24.937711) (end 20.365634 -24.937711) (width 0.2) (layer "B.Cu") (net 4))
 (segment (start -12.265281 -27.813683) (end -9.388349 -24.936751) (width 0.2) (layer "B.Cu") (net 4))
 (segment (start -2.998337 -24.936751) (end -2.997377 -24.937711) (width 0.2) (layer "B.Cu") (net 4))
 (segment (start -9.388349 -24.936751) (end -2.998337 -24.936751) (width 0.2) (layer "B.Cu") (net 4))
 (segment (start 53.337606 -26.175136) (end 56.928406 -22.584336) (width 0.2) (layer "B.Cu") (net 4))
 (segment (start 25.659431 -29.100136) (end 36.258461 -29.100136) (width 0.2) (layer "B.Cu") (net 19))
 (segment (start 53.006235 -25.375136) (end 56.597035 -21.784336) (width 0.2) (layer "B.Cu") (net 19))
 (segment (start 6.186966 -17.89527) (end 6.186966 -20.908754) (width 0.2) (layer "B.Cu") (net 19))
 (segment (start 56.597035 -21.784336) (end 84.902964 -21.784336) (width 0.2) (layer "B.Cu") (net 19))
 (segment (start 6.186966 -20.908754) (end 9.415923 -24.137711) (width 0.2) (layer "B.Cu") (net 19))
 (segment (start 87.242646 -33.684336) (end 90.018946 -36.460636) (width 0.2) (layer "B.Cu") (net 19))
 (segment (start 39.983461 -25.375136) (end 53.006235 -25.375136) (width 0.2) (layer "B.Cu") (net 19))
 (segment (start 20.697006 -24.137711) (end 25.659431 -29.100136) (width 0.2) (layer "B.Cu") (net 19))
 (segment (start 36.258461 -29.100136) (end 39.983461 -25.375136) (width 0.2) (layer "B.Cu") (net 19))
 (segment (start 87.242646 -24.124018) (end 87.242646 -33.684336) (width 0.2) (layer "B.Cu") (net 19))
 (segment (start 84.902964 -21.784336) (end 87.242646 -24.124018) (width 0.2) (layer "B.Cu") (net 19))
 (segment (start 9.415923 -24.137711) (end 20.697006 -24.137711) (width 0.2) (layer "B.Cu") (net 19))
 (segment (start 39.983461 -41.875136) (end 52.924147 -41.875136) (width 0.2) (layer "B.Cu") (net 13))
 (segment (start 60.774147 -34.025136) (end 69.589833 -34.025136) (width 0.2) (layer "B.Cu") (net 13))
 (segment (start 24.029648 -43.970353) (end 25.425117 -45.365821) (width 0.2) (layer "B.Cu") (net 13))
 (segment (start 72.234333 -31.380636) (end 74.778946 -31.380636) (width 0.2) (layer "B.Cu") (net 13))
 (segment (start 5.323423 -37.386141) (end 8.55238 -40.615098) (width 0.2) (layer "B.Cu") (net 13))
 (segment (start 25.425117 -45.365821) (end 25.659431 -45.600136) (width 0.2) (layer "B.Cu") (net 13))
 (segment (start 52.924147 -41.875136) (end 60.774147 -34.025136) (width 0.2) (layer "B.Cu") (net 13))
 (segment (start 20.674393 -40.615098) (end 24.029648 -43.970353) (width 0.2) (layer "B.Cu") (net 13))
 (segment (start 36.258461 -45.600136) (end 39.983461 -41.875136) (width 0.2) (layer "B.Cu") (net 13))
 (segment (start 8.55238 -40.615098) (end 20.674393 -40.615098) (width 0.2) (layer "B.Cu") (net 13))
 (segment (start 5.323423 -34.372657) (end 5.323423 -37.386141) (width 0.2) (layer "B.Cu") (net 13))
 (segment (start 69.589833 -34.025136) (end 72.234333 -31.380636) (width 0.2) (layer "B.Cu") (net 13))
 (segment (start 25.659431 -45.600136) (end 36.258461 -45.600136) (width 0.2) (layer "B.Cu") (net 13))
 (segment (start 25.659431 -62.100136) (end 36.258461 -62.100136) (width 0.2) (layer "B.Cu") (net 10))
 (segment (start 4.45988 -53.863528) (end 7.688837 -57.092485) (width 0.2) (layer "B.Cu") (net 10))
 (segment (start 69.589833 -50.525136) (end 73.602646 -46.512323) (width 0.2) (layer "B.Cu") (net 10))
 (segment (start 39.983461 -58.375136) (end 53.006236 -58.375136) (width 0.2) (layer "B.Cu") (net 10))
 (segment (start 60.856236 -50.525136) (end 69.589833 -50.525136) (width 0.2) (layer "B.Cu") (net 10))
 (segment (start 73.602646 -46.512323) (end 73.602646 -42.716936) (width 0.2) (layer "B.Cu") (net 10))
 (segment (start 4.45988 -50.850044) (end 4.45988 -53.863528) (width 0.2) (layer "B.Cu") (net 10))
 (segment (start 20.65178 -57.092485) (end 25.659431 -62.100136) (width 0.2) (layer "B.Cu") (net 10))
 (segment (start 36.258461 -62.100136) (end 39.983461 -58.375136) (width 0.2) (layer "B.Cu") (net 10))
 (segment (start 7.688837 -57.092485) (end 20.65178 -57.092485) (width 0.2) (layer "B.Cu") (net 10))
 (segment (start 73.602646 -42.716936) (end 74.778946 -41.540636) (width 0.2) (layer "B.Cu") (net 10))
 (segment (start 53.006236 -58.375136) (end 60.856236 -50.525136) (width 0.2) (layer "B.Cu") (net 10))
 (segment (start 25.825117 -28.700136) (end 36.092775 -28.700136) (width 0.2) (layer "B.Cu") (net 20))
 (segment (start 54.657843 -23.157843) (end 56.43135 -21.384336) (width 0.2) (layer "B.Cu") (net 20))
 (segment (start 52.84055 -24.975136) (end 54.657843 -23.157843) (width 0.2) (layer "B.Cu") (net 20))
 (segment (start 54.657843 -23.157843) (end 54.75 -23.065685) (width 0.2) (layer "B.Cu") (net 20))
 (segment (start 36.092775 -28.700136) (end 39.817775 -24.975136) (width 0.2) (layer "B.Cu") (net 20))
 (segment (start 22.683946 -25.558965) (end 25.825117 -28.700136) (width 0.2) (layer "B.Cu") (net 20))
 (segment (start 85.06865 -21.384336) (end 87.642646 -23.958332) (width 0.2) (layer "B.Cu") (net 20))
 (segment (start 87.642646 -31.544336) (end 90.018946 -33.920636) (width 0.2) (layer "B.Cu") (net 20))
 (segment (start 56.43135 -21.384336) (end 85.06865 -21.384336) (width 0.2) (layer "B.Cu") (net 20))
 (segment (start 22.683946 -22.885636) (end 22.683946 -25.558965) (width 0.2) (layer "B.Cu") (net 20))
 (segment (start 87.642646 -23.958332) (end 87.642646 -31.544336) (width 0.2) (layer "B.Cu") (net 20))
 (segment (start 39.817775 -24.975136) (end 52.84055 -24.975136) (width 0.2) (layer "B.Cu") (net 20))
 (segment (start 36.092775 -45.200136) (end 25.825117 -45.200136) (width 0.2) (layer "B.Cu") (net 3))
 (segment (start 74.208647 -28.840636) (end 69.424147 -33.625136) (width 0.2) (layer "B.Cu") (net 3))
 (segment (start 60.608461 -33.625136) (end 52.758461 -41.475136) (width 0.2) (layer "B.Cu") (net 3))
 (segment (start 69.424147 -33.625136) (end 60.608461 -33.625136) (width 0.2) (layer "B.Cu") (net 3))
 (segment (start 39.817775 -41.475136) (end 36.092775 -45.200136) (width 0.2) (layer "B.Cu") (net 3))
 (segment (start 22.683946 -42.058965) (end 22.683946 -39.385636) (width 0.2) (layer "B.Cu") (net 3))
 (segment (start 52.758461 -41.475136) (end 39.817775 -41.475136) (width 0.2) (layer "B.Cu") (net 3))
 (segment (start 25.825117 -45.200136) (end 22.683946 -42.058965) (width 0.2) (layer "B.Cu") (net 3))
 (segment (start 74.778946 -28.840636) (end 74.208647 -28.840636) (width 0.2) (layer "B.Cu") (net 3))
 (segment (start 36.092775 -61.700136) (end 39.817775 -57.975136) (width 0.2) (layer "B.Cu") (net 11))
 (segment (start 60.69055 -50.125136) (end 69.424147 -50.125136) (width 0.2) (layer "B.Cu") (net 11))
 (segment (start 73.202646 -46.346637) (end 73.202646 -40.576936) (width 0.2) (layer "B.Cu") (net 11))
 (segment (start 22.683946 -58.558965) (end 25.825117 -61.700136) (width 0.2) (layer "B.Cu") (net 11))
 (segment (start 25.825117 -61.700136) (end 36.092775 -61.700136) (width 0.2) (layer "B.Cu") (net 11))
 (segment (start 52.84055 -57.975136) (end 60.69055 -50.125136) (width 0.2) (layer "B.Cu") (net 11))
 (segment (start 39.817775 -57.975136) (end 52.84055 -57.975136) (width 0.2) (layer "B.Cu") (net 11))
 (segment (start 73.202646 -40.576936) (end 74.778946 -39.000636) (width 0.2) (layer "B.Cu") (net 11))
 (segment (start 22.683946 -55.885636) (end 22.683946 -58.558965) (width 0.2) (layer "B.Cu") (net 11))
 (segment (start 69.424147 -50.125136) (end 73.202646 -46.346637) (width 0.2) (layer "B.Cu") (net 11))
 (segment (start 56.265664 -20.984336) (end 85.234336 -20.984336) (width 0.2) (layer "B.Cu") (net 21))
 (segment (start 88.042646 -29.404336) (end 90.018946 -31.380636) (width 0.2) (layer "B.Cu") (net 21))
 (segment (start 39.183946 -21.433965) (end 42.325117 -24.575136) (width 0.2) (layer "B.Cu") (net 21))
 (segment (start 52.674864 -24.575136) (end 56.265664 -20.984336) (width 0.2) (layer "B.Cu") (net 21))
 (segment (start 85.234336 -20.984336) (end 88.042646 -23.792646) (width 0.2) (layer "B.Cu") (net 21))
 (segment (start 42.325117 -24.575136) (end 52.674864 -24.575136) (width 0.2) (layer "B.Cu") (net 21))
 (segment (start 39.183946 -18.760636) (end 39.183946 -21.433965) (width 0.2) (layer "B.Cu") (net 21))
 (segment (start 88.042646 -23.792646) (end 88.042646 -29.404336) (width 0.2) (layer "B.Cu") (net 21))
 (segment (start 52.592775 -41.075136) (end 60.442775 -33.225136) (width 0.2) (layer "B.Cu") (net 14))
 (segment (start 42.325117 -41.075136) (end 52.592775 -41.075136) (width 0.2) (layer "B.Cu") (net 14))
 (segment (start 73.602646 -27.476936) (end 74.778946 -26.300636) (width 0.2) (layer "B.Cu") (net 14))
 (segment (start 39.183946 -37.933965) (end 42.325117 -41.075136) (width 0.2) (layer "B.Cu") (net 14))
 (segment (start 73.602646 -28.880951) (end 73.602646 -27.476936) (width 0.2) (layer "B.Cu") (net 14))
 (segment (start 39.183946 -35.260636) (end 39.183946 -37.933965) (width 0.2) (layer "B.Cu") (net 14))
 (segment (start 69.258461 -33.225136) (end 73.602646 -28.880951) (width 0.2) (layer "B.Cu") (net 14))
 (segment (start 60.442775 -33.225136) (end 69.258461 -33.225136) (width 0.2) (layer "B.Cu") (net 14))
 (segment (start 72.75 -38.489582) (end 74.778946 -36.460636) (width 0.2) (layer "B.Cu") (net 2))
 (segment (start 72.75 -46.233597) (end 72.75 -38.489582) (width 0.2) (layer "B.Cu") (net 2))
 (segment (start 69.258461 -49.725136) (end 72.75 -46.233597) (width 0.2) (layer "B.Cu") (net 2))
 (segment (start 60.524864 -49.725136) (end 69.258461 -49.725136) (width 0.2) (layer "B.Cu") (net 2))
 (segment (start 39.183946 -51.760636) (end 39.183946 -54.433965) (width 0.2) (layer "B.Cu") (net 2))
 (segment (start 39.183946 -54.433965) (end 42.325117 -57.575136) (width 0.2) (layer "B.Cu") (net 2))
 (segment (start 52.674864 -57.575136) (end 60.524864 -49.725136) (width 0.2) (layer "B.Cu") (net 2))
 (segment (start 42.325117 -57.575136) (end 52.674864 -57.575136) (width 0.2) (layer "B.Cu") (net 2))
 (segment (start 55.683946 -27.010636) (end 55.683946 -29.683965) (width 0.2) (layer "B.Cu") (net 15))
 (segment (start 69.092775 -32.825136) (end 73.202646 -28.715265) (width 0.2) (layer "B.Cu") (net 15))
 (segment (start 73.202646 -25.336936) (end 74.778946 -23.760636) (width 0.2) (layer "B.Cu") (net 15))
 (segment (start 73.202646 -28.715265) (end 73.202646 -25.336936) (width 0.2) (layer "B.Cu") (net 15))
 (segment (start 55.683946 -29.683965) (end 58.825117 -32.825136) (width 0.2) (layer "B.Cu") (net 15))
 (segment (start 58.825117 -32.825136) (end 69.092775 -32.825136) (width 0.2) (layer "B.Cu") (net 15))
 (segment (start 69.092775 -49.325136) (end 72.35 -46.067911) (width 0.2) (layer "B.Cu") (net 12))
 (segment (start 58.825117 -49.325136) (end 69.092775 -49.325136) (width 0.2) (layer "B.Cu") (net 12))
 (segment (start 72.35 -36.349582) (end 74.778946 -33.920636) (width 0.2) (layer "B.Cu") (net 12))
 (segment (start 55.683946 -46.183965) (end 58.825117 -49.325136) (width 0.2) (layer "B.Cu") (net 12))
 (segment (start 72.35 -46.067911) (end 72.35 -36.349582) (width 0.2) (layer "B.Cu") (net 12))
 (segment (start 55.683946 -43.510636) (end 55.683946 -46.183965) (width 0.2) (layer "B.Cu") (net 12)))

